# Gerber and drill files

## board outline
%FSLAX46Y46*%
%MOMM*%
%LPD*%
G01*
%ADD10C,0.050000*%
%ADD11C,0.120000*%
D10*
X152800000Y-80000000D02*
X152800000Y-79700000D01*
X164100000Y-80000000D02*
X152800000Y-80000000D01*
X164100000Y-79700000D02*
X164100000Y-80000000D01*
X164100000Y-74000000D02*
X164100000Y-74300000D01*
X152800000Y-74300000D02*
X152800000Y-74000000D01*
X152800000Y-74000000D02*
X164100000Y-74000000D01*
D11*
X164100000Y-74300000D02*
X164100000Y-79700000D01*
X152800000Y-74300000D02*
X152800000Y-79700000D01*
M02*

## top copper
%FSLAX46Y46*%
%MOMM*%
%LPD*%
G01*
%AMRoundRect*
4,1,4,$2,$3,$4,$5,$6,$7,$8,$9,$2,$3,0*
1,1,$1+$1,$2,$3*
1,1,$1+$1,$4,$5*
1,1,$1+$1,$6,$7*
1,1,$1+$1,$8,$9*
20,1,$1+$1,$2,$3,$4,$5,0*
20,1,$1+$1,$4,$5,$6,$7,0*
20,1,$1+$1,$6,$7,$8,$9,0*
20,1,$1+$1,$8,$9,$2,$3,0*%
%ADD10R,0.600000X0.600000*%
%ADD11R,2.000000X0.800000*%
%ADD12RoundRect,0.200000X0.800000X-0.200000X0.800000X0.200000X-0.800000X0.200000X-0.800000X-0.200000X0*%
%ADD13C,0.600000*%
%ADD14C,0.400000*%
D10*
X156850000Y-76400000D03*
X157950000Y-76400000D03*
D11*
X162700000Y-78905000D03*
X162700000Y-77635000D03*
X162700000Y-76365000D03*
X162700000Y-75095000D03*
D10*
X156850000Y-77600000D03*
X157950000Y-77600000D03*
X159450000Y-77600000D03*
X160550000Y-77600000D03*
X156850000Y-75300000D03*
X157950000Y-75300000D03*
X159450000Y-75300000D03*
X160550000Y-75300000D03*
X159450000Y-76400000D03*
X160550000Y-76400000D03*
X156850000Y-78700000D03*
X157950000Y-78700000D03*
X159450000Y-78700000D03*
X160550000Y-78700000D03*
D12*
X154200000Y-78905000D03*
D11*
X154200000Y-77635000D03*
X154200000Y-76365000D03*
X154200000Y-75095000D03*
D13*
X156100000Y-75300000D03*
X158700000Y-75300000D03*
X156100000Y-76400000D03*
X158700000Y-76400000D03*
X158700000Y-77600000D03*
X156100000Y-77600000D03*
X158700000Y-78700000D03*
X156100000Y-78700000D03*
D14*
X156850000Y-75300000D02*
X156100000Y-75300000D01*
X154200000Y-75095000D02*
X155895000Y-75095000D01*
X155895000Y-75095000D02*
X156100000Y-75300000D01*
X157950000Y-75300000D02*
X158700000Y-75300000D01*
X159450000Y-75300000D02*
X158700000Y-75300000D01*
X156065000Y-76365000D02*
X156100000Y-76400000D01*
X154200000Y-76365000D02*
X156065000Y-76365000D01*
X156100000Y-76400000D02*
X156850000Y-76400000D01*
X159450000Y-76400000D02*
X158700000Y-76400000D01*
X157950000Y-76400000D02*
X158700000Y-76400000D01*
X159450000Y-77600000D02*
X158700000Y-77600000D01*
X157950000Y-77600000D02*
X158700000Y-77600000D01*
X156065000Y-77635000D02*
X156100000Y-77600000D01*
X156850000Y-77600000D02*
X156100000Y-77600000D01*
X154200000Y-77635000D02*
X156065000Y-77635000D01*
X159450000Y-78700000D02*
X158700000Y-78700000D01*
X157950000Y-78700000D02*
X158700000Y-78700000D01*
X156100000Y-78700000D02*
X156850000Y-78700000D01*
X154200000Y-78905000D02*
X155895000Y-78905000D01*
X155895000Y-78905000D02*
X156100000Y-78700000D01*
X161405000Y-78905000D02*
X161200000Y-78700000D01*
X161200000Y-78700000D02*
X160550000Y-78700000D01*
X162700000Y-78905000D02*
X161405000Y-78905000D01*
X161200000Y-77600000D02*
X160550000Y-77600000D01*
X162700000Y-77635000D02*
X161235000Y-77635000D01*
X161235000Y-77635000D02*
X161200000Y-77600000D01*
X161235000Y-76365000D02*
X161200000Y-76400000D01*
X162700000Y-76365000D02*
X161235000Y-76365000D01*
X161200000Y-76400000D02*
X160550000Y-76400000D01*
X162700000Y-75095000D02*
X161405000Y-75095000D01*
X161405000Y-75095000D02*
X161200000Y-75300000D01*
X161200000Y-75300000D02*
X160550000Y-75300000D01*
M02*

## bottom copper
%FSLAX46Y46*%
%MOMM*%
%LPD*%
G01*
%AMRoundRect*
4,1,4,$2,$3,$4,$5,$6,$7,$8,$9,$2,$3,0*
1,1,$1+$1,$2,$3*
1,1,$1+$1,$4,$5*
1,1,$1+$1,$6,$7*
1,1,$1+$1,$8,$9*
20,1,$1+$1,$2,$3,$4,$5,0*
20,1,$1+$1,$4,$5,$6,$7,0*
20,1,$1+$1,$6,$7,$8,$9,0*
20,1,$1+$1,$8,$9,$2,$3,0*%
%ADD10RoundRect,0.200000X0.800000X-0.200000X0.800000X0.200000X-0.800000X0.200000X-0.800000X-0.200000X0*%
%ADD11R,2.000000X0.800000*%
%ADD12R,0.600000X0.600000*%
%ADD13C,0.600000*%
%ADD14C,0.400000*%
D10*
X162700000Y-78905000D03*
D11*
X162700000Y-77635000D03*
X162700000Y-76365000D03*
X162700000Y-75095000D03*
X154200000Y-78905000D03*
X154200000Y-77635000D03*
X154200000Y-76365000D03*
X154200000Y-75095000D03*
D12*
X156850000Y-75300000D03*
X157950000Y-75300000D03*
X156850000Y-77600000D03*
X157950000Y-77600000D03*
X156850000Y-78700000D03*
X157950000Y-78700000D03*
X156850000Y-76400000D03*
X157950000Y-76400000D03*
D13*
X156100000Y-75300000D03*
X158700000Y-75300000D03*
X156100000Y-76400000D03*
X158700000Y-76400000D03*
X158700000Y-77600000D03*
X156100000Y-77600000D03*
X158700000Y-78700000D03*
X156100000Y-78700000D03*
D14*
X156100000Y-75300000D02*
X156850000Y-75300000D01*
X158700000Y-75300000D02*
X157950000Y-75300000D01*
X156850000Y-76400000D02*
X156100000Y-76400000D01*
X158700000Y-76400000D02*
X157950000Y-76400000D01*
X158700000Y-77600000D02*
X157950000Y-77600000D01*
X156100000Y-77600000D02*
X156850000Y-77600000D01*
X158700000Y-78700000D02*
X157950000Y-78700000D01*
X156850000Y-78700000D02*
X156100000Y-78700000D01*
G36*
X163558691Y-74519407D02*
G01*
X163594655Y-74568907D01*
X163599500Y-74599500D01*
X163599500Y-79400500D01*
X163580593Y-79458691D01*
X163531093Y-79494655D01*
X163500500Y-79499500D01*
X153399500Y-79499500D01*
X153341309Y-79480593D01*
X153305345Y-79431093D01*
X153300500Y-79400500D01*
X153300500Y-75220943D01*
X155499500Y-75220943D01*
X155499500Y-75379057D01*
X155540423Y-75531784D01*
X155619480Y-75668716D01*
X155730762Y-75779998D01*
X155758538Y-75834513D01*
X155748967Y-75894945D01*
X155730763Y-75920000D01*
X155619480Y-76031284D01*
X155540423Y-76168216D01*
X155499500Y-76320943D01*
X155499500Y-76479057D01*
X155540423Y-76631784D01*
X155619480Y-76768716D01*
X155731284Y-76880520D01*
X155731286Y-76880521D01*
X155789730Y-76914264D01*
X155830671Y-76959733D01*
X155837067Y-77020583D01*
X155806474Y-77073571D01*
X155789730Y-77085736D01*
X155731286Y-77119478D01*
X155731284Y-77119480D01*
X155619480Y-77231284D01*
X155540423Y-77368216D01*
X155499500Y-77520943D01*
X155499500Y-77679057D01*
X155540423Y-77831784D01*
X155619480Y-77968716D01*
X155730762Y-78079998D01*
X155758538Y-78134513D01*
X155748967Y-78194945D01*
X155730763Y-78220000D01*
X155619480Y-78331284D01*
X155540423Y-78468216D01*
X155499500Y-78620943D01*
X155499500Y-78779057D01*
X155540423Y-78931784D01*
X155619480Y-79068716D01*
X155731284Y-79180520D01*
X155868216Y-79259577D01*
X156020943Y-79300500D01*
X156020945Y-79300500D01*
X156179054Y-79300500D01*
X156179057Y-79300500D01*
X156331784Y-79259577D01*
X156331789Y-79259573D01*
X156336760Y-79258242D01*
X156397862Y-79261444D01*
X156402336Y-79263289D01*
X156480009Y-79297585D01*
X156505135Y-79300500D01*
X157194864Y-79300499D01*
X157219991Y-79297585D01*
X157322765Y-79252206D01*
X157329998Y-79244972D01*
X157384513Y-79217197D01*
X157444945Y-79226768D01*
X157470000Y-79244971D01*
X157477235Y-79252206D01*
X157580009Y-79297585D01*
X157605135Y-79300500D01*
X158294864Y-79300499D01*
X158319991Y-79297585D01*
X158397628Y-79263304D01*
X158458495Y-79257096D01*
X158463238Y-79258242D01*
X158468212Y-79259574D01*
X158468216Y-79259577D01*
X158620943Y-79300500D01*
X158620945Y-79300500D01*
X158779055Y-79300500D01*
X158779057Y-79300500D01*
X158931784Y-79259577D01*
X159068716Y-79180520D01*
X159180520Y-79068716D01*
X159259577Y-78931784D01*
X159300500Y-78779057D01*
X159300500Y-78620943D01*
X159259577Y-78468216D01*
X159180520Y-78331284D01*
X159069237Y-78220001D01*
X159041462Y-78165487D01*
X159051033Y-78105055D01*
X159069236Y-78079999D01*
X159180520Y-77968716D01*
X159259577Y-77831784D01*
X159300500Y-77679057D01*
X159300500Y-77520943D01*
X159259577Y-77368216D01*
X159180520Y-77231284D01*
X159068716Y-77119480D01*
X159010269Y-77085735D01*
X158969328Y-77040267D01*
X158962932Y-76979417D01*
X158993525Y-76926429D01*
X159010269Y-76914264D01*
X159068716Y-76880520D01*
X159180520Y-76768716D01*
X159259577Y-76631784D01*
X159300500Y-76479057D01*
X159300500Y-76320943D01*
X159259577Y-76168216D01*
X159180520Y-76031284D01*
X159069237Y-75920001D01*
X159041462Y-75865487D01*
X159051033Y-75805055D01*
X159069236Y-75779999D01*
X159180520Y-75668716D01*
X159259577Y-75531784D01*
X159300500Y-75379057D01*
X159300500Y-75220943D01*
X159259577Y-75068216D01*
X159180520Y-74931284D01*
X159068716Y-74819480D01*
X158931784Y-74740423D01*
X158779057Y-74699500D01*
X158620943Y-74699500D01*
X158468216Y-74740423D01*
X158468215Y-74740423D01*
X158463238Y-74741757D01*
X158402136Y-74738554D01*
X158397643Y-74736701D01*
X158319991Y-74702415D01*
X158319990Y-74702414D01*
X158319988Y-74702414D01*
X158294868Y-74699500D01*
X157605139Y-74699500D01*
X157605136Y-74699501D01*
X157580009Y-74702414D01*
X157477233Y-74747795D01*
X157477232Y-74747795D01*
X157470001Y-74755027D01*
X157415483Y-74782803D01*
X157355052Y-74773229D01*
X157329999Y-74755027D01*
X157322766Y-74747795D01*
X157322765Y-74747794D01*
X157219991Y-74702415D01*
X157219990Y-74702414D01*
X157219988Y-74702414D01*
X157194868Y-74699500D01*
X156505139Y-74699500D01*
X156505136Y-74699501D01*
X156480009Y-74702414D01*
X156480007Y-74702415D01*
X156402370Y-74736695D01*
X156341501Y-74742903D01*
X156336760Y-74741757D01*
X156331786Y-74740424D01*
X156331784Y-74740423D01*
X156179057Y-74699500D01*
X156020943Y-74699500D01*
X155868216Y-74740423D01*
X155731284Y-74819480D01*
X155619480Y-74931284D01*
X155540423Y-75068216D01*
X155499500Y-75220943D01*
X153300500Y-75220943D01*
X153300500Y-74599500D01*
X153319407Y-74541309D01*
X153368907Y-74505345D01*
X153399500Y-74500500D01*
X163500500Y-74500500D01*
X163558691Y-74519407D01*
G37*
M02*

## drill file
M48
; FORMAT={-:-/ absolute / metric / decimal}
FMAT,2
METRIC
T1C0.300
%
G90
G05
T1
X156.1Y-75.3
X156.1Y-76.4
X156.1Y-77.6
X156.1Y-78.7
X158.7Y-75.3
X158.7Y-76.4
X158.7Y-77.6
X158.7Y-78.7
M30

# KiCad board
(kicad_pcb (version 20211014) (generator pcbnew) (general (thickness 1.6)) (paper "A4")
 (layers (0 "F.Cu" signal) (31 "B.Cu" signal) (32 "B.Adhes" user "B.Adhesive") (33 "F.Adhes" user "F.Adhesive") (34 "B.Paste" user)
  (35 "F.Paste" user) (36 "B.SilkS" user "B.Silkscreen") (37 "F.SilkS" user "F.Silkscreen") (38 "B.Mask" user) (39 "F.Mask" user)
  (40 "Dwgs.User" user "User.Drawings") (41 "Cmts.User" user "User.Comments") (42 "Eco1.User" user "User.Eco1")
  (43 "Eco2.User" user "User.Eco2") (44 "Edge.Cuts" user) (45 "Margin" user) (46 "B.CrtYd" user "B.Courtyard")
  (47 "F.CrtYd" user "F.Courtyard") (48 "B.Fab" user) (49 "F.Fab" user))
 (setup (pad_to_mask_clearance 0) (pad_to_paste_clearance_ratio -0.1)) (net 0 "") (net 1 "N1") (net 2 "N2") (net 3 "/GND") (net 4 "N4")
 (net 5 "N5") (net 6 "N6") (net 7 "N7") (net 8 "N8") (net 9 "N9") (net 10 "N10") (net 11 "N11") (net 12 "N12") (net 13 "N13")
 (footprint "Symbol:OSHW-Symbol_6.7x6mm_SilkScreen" (layer "F.Cu") (at 147 76.2)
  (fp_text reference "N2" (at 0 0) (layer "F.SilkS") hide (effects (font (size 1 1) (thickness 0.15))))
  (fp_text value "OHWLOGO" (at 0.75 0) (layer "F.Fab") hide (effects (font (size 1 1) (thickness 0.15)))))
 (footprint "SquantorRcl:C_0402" (layer "F.Cu") (at 157.4 76.4)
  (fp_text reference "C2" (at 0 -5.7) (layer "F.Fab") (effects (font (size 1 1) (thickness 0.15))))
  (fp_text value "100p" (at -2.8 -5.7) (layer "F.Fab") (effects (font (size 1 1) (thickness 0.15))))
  (pad "1" smd rect (at -0.55 0) (size 0.6 0.6) (layers "F.Cu" "F.Paste" "F.Mask") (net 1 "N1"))
  (pad "2" smd rect (at 0.55 0) (size 0.6 0.6) (layers "F.Cu" "F.Paste" "F.Mask") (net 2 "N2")))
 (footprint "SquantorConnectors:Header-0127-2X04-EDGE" (layer "F.Cu") (at 161.6 77 90)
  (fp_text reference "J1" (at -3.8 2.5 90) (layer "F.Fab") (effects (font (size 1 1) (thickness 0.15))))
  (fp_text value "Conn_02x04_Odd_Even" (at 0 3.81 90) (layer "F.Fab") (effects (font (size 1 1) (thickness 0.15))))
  (fp_line (start 2.7 2.5) (end -2.7 2.5) (layer "Edge.Cuts") (width 0.12))
  (pad "1" smd roundrect (at -1.905 1.1 90) (size 0.8 2) (layers "B.Cu" "B.Paste" "B.Mask") (roundrect_rratio 0.25) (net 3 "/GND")
   (zone_connect 2))
  (pad "2" smd rect (at -1.905 1.1 90) (size 0.8 2) (layers "F.Cu" "F.Paste" "F.Mask") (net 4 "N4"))
  (pad "3" smd rect (at -0.635 1.1 90) (size 0.8 2) (layers "B.Cu" "B.Paste" "B.Mask") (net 3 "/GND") (zone_connect 2))
  (pad "4" smd rect (at -0.635 1.1 90) (size 0.8 2) (layers "F.Cu" "F.Paste" "F.Mask") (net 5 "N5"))
  (pad "5" smd rect (at 0.635 1.1 90) (size 0.8 2) (layers "B.Cu" "B.Paste" "B.Mask") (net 3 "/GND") (zone_connect 2))
  (pad "6" smd rect (at 0.635 1.1 90) (size 0.8 2) (layers "F.Cu" "F.Paste" "F.Mask") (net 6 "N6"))
  (pad "7" smd rect (at 1.905 1.1 90) (size 0.8 2) (layers "B.Cu" "B.Paste" "B.Mask") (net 3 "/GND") (zone_connect 2))
  (pad "8" smd rect (at 1.905 1.1 90) (size 0.8 2) (layers "F.Cu" "F.Paste" "F.Mask") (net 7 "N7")))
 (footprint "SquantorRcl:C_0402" (layer "F.Cu") (at 157.4 77.6)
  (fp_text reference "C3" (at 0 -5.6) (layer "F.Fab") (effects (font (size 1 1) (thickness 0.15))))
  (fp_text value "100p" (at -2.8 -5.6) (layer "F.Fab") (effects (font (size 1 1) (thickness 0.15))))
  (pad "1" smd rect (at -0.55 0) (size 0.6 0.6) (layers "F.Cu" "F.Paste" "F.Mask") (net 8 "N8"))
  (pad "2" smd rect (at 0.55 0) (size 0.6 0.6) (layers "F.Cu" "F.Paste" "F.Mask") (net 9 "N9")))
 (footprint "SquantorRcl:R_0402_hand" (layer "F.Cu") (at 160 77.6)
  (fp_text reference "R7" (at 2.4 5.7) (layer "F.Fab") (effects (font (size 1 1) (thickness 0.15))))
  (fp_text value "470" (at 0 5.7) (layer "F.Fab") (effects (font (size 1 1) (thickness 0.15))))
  (pad "1" smd rect (at -0.55 0) (size 0.6 0.6) (layers "F.Cu" "F.Paste" "F.Mask") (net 9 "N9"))
  (pad "2" smd rect (at 0.55 0) (size 0.6 0.6) (layers "F.Cu" "F.Paste" "F.Mask") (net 5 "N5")))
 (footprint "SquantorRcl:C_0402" (layer "F.Cu") (at 157.4 75.3)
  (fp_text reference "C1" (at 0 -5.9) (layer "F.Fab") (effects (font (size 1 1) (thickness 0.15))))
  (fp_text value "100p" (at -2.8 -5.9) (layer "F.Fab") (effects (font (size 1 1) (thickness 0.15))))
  (pad "1" smd rect (at -0.55 0) (size 0.6 0.6) (layers "F.Cu" "F.Paste" "F.Mask") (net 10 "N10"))
  (pad "2" smd rect (at 0.55 0) (size 0.6 0.6) (layers "F.Cu" "F.Paste" "F.Mask") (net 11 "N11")))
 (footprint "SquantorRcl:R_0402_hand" (layer "F.Cu") (at 160 75.3)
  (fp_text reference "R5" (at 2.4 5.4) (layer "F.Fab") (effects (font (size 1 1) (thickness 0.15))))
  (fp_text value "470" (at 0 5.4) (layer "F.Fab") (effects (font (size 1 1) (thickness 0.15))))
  (pad "1" smd rect (at -0.55 0) (size 0.6 0.6) (layers "F.Cu" "F.Paste" "F.Mask") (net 11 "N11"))
  (pad "2" smd rect (at 0.55 0) (size 0.6 0.6) (layers "F.Cu" "F.Paste" "F.Mask") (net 7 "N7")))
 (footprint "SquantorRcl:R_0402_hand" (layer "F.Cu") (at 160 76.4)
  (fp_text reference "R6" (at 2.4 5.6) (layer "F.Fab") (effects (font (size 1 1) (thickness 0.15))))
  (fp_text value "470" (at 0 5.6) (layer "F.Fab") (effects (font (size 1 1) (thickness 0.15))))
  (pad "1" smd rect (at -0.55 0) (size 0.6 0.6) (layers "F.Cu" "F.Paste" "F.Mask") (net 2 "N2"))
  (pad "2" smd rect (at 0.55 0) (size 0.6 0.6) (layers "F.Cu" "F.Paste" "F.Mask") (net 6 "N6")))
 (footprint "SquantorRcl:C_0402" (layer "F.Cu") (at 157.4 78.7)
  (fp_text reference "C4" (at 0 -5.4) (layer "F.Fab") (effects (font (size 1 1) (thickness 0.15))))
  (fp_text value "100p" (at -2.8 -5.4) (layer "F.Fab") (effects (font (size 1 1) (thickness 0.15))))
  (pad "1" smd rect (at -0.55 0) (size 0.6 0.6) (layers "F.Cu" "F.Paste" "F.Mask") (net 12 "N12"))
  (pad "2" smd rect (at 0.55 0) (size 0.6 0.6) (layers "F.Cu" "F.Paste" "F.Mask") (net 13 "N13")))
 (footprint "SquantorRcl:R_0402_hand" (layer "F.Cu") (at 160 78.7)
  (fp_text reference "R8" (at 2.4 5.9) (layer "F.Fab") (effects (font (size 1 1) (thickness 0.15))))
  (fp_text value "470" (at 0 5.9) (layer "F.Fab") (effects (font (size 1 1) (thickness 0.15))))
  (pad "1" smd rect (at -0.55 0) (size 0.6 0.6) (layers "F.Cu" "F.Paste" "F.Mask") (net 13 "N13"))
  (pad "2" smd rect (at 0.55 0) (size 0.6 0.6) (layers "F.Cu" "F.Paste" "F.Mask") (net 4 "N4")))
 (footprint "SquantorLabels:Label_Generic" (layer "B.Cu") (at 159.6 76.2 -90)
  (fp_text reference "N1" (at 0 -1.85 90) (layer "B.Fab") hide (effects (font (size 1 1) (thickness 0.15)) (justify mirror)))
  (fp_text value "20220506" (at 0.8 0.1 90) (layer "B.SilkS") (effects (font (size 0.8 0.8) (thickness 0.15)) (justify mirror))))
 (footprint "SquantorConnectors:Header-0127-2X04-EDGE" (layer "B.Cu") (at 155.3 77 90)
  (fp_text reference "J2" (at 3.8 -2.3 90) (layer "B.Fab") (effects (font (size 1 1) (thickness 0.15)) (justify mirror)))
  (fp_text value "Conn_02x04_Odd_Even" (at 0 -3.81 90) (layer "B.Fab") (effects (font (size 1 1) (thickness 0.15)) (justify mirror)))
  (fp_line (start 2.7 -2.5) (end -2.7 -2.5) (layer "Edge.Cuts") (width 0.12))
  (pad "1" smd roundrect (at -1.905 -1.1 90) (size 0.8 2) (layers "F.Cu" "F.Paste" "F.Mask") (roundrect_rratio 0.25) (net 12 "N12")
   (zone_connect 2))
  (pad "2" smd rect (at -1.905 -1.1 90) (size 0.8 2) (layers "B.Cu" "B.Paste" "B.Mask") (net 3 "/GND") (zone_connect 2))
  (pad "3" smd rect (at -0.635 -1.1 90) (size 0.8 2) (layers "F.Cu" "F.Paste" "F.Mask") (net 8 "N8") (zone_connect 2))
  (pad "4" smd rect (at -0.635 -1.1 90) (size 0.8 2) (layers "B.Cu" "B.Paste" "B.Mask") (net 3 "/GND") (zone_connect 2))
  (pad "5" smd rect (at 0.635 -1.1 90) (size 0.8 2) (layers "F.Cu" "F.Paste" "F.Mask") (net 1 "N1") (zone_connect 2))
  (pad "6" smd rect (at 0.635 -1.1 90) (size 0.8 2) (layers "B.Cu" "B.Paste" "B.Mask") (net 3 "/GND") (zone_connect 2))
  (pad "7" smd rect (at 1.905 -1.1 90) (size 0.8 2) (layers "F.Cu" "F.Paste" "F.Mask") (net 10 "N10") (zone_connect 2))
  (pad "8" smd rect (at 1.905 -1.1 90) (size 0.8 2) (layers "B.Cu" "B.Paste" "B.Mask") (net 3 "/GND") (zone_connect 2)))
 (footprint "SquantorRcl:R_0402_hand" (layer "B.Cu") (at 157.4 75.3)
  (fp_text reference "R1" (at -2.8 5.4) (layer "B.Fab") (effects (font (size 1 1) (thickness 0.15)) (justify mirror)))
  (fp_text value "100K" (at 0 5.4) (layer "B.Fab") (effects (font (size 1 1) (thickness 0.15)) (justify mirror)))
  (pad "1" smd rect (at -0.55 0) (size 0.6 0.6) (layers "B.Cu" "B.Paste" "B.Mask") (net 10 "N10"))
  (pad "2" smd rect (at 0.55 0) (size 0.6 0.6) (layers "B.Cu" "B.Paste" "B.Mask") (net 11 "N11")))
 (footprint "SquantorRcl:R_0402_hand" (layer "B.Cu") (at 157.4 77.6)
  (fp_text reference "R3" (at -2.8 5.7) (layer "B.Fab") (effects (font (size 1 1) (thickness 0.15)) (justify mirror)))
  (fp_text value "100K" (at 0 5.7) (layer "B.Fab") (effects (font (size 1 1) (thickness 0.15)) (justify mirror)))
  (pad "1" smd rect (at -0.55 0) (size 0.6 0.6) (layers "B.Cu" "B.Paste" "B.Mask") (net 8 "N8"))
  (pad "2" smd rect (at 0.55 0) (size 0.6 0.6) (layers "B.Cu" "B.Paste" "B.Mask") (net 9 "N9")))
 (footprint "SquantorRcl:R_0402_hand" (layer "B.Cu") (at 157.4 78.7)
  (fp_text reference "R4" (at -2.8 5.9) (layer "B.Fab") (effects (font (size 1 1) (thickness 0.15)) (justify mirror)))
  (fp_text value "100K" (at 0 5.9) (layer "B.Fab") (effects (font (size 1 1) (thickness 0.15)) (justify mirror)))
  (pad "1" smd rect (at -0.55 0) (size 0.6 0.6) (layers "B.Cu" "B.Paste" "B.Mask") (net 12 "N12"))
  (pad "2" smd rect (at 0.55 0) (size 0.6 0.6) (layers "B.Cu" "B.Paste" "B.Mask") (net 13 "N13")))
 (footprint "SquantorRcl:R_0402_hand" (layer "B.Cu") (at 157.4 76.4)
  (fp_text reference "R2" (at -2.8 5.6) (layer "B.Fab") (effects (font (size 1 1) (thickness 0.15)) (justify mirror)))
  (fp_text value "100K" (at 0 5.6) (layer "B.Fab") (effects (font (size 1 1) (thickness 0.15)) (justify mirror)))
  (pad "1" smd rect (at -0.55 0) (size 0.6 0.6) (layers "B.Cu" "B.Paste" "B.Mask") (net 1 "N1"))
  (pad "2" smd rect (at 0.55 0) (size 0.6 0.6) (layers "B.Cu" "B.Paste" "B.Mask") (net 2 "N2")))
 (gr_line (start 152.8 80) (end 152.8 79.7) (layer "Edge.Cuts") (width 0.05))
 (gr_line (start 164.1 80) (end 152.8 80) (layer "Edge.Cuts") (width 0.05))
 (gr_line (start 164.1 79.7) (end 164.1 80) (layer "Edge.Cuts") (width 0.05))
 (gr_line (start 164.1 74) (end 164.1 74.3) (layer "Edge.Cuts") (width 0.05))
 (gr_line (start 152.8 74.3) (end 152.8 74) (layer "Edge.Cuts") (width 0.05))
 (gr_line (start 152.8 74) (end 164.1 74) (layer "Edge.Cuts") (width 0.05))
 (segment (start 156.85 75.3) (end 156.1 75.3) (width 0.4) (layer "F.Cu") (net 10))
 (segment (start 154.2 75.095) (end 155.895 75.095) (width 0.4) (layer "F.Cu") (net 10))
 (segment (start 155.895 75.095) (end 156.1 75.3) (width 0.4) (layer "F.Cu") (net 10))
 (via (at 156.1 75.3) (size 0.6) (drill 0.3) (layers "F.Cu" "B.Cu") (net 10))
 (segment (start 156.1 75.3) (end 156.85 75.3) (width 0.4) (layer "B.Cu") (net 10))
 (segment (start 157.95 75.3) (end 158.7 75.3) (width 0.4) (layer "F.Cu") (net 11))
 (segment (start 159.45 75.3) (end 158.7 75.3) (width 0.4) (layer "F.Cu") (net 11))
 (via (at 158.7 75.3) (size 0.6) (drill 0.3) (layers "F.Cu" "B.Cu") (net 11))
 (segment (start 158.7 75.3) (end 157.95 75.3) (width 0.4) (layer "B.Cu") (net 11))
 (segment (start 156.065 76.365) (end 156.1 76.4) (width 0.4) (layer "F.Cu") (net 1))
 (segment (start 154.2 76.365) (end 156.065 76.365) (width 0.4) (layer "F.Cu") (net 1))
 (segment (start 156.1 76.4) (end 156.85 76.4) (width 0.4) (layer "F.Cu") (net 1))
 (via (at 156.1 76.4) (size 0.6) (drill 0.3) (layers "F.Cu" "B.Cu") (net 1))
 (segment (start 156.85 76.4) (end 156.1 76.4) (width 0.4) (layer "B.Cu") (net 1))
 (segment (start 159.45 76.4) (end 158.7 76.4) (width 0.4) (layer "F.Cu") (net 2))
 (segment (start 157.95 76.4) (end 158.7 76.4) (width 0.4) (layer "F.Cu") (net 2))
 (via (at 158.7 76.4) (size 0.6) (drill 0.3) (layers "F.Cu" "B.Cu") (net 2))
 (segment (start 158.7 76.4) (end 157.95 76.4) (width 0.4) (layer "B.Cu") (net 2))
 (segment (start 159.45 77.6) (end 158.7 77.6) (width 0.4) (layer "F.Cu") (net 9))
 (segment (start 157.95 77.6) (end 158.7 77.6) (width 0.4) (layer "F.Cu") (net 9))
 (via (at 158.7 77.6) (size 0.6) (drill 0.3) (layers "F.Cu" "B.Cu") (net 9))
 (segment (start 158.7 77.6) (end 157.95 77.6) (width 0.4) (layer "B.Cu") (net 9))
 (segment (start 156.065 77.635) (end 156.1 77.6) (width 0.4) (layer "F.Cu") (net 8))
 (segment (start 156.85 77.6) (end 156.1 77.6) (width 0.4) (layer "F.Cu") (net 8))
 (segment (start 154.2 77.635) (end 156.065 77.635) (width 0.4) (layer "F.Cu") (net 8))
 (via (at 156.1 77.6) (size 0.6) (drill 0.3) (layers "F.Cu" "B.Cu") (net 8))
 (segment (start 156.1 77.6) (end 156.85 77.6) (width 0.4) (layer "B.Cu") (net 8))
 (segment (start 159.45 78.7) (end 158.7 78.7) (width 0.4) (layer "F.Cu") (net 13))
 (segment (start 157.95 78.7) (end 158.7 78.7) (width 0.4) (layer "F.Cu") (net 13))
 (via (at 158.7 78.7) (size 0.6) (drill 0.3) (layers "F.Cu" "B.Cu") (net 13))
 (segment (start 158.7 78.7) (end 157.95 78.7) (width 0.4) (layer "B.Cu") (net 13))
 (segment (start 156.1 78.7) (end 156.85 78.7) (width 0.4) (layer "F.Cu") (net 12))
 (segment (start 154.2 78.905) (end 155.895 78.905) (width 0.4) (layer "F.Cu") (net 12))
 (segment (start 155.895 78.905) (end 156.1 78.7) (width 0.4) (layer "F.Cu") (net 12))
 (via (at 156.1 78.7) (size 0.6) (drill 0.3) (layers "F.Cu" "B.Cu") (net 12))
 (segment (start 156.85 78.7) (end 156.1 78.7) (width 0.4) (layer "B.Cu") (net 12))
 (segment (start 161.405 78.905) (end 161.2 78.7) (width 0.4) (layer "F.Cu") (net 4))
 (segment (start 161.2 78.7) (end 160.55 78.7) (width 0.4) (layer "F.Cu") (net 4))
 (segment (start 162.7 78.905) (end 161.405 78.905) (width 0.4) (layer "F.Cu") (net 4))
 (segment (start 161.2 77.6) (end 160.55 77.6) (width 0.4) (layer "F.Cu") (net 5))
 (segment (start 162.7 77.635) (end 161.235 77.635) (width 0.4) (layer "F.Cu") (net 5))
 (segment (start 161.235 77.635) (end 161.2 77.6) (width 0.4) (layer "F.Cu") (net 5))
 (segment (start 161.235 76.365) (end 161.2 76.4) (width 0.4) (layer "F.Cu") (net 6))
 (segment (start 162.7 76.365) (end 161.235 76.365) (width 0.4) (layer "F.Cu") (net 6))
 (segment (start 161.2 76.4) (end 160.55 76.4) (width 0.4) (layer "F.Cu") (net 6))
 (segment (start 162.7 75.095) (end 161.405 75.095) (width 0.4) (layer "F.Cu") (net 7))
 (segment (start 161.405 75.095) (end 161.2 75.3) (width 0.4) (layer "F.Cu") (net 7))
 (segment (start 161.2 75.3) (end 160.55 75.3) (width 0.4) (layer "F.Cu") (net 7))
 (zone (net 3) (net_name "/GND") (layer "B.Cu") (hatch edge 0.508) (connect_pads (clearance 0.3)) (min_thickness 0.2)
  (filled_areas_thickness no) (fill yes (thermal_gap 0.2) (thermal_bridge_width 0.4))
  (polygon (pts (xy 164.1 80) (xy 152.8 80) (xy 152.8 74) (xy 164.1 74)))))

